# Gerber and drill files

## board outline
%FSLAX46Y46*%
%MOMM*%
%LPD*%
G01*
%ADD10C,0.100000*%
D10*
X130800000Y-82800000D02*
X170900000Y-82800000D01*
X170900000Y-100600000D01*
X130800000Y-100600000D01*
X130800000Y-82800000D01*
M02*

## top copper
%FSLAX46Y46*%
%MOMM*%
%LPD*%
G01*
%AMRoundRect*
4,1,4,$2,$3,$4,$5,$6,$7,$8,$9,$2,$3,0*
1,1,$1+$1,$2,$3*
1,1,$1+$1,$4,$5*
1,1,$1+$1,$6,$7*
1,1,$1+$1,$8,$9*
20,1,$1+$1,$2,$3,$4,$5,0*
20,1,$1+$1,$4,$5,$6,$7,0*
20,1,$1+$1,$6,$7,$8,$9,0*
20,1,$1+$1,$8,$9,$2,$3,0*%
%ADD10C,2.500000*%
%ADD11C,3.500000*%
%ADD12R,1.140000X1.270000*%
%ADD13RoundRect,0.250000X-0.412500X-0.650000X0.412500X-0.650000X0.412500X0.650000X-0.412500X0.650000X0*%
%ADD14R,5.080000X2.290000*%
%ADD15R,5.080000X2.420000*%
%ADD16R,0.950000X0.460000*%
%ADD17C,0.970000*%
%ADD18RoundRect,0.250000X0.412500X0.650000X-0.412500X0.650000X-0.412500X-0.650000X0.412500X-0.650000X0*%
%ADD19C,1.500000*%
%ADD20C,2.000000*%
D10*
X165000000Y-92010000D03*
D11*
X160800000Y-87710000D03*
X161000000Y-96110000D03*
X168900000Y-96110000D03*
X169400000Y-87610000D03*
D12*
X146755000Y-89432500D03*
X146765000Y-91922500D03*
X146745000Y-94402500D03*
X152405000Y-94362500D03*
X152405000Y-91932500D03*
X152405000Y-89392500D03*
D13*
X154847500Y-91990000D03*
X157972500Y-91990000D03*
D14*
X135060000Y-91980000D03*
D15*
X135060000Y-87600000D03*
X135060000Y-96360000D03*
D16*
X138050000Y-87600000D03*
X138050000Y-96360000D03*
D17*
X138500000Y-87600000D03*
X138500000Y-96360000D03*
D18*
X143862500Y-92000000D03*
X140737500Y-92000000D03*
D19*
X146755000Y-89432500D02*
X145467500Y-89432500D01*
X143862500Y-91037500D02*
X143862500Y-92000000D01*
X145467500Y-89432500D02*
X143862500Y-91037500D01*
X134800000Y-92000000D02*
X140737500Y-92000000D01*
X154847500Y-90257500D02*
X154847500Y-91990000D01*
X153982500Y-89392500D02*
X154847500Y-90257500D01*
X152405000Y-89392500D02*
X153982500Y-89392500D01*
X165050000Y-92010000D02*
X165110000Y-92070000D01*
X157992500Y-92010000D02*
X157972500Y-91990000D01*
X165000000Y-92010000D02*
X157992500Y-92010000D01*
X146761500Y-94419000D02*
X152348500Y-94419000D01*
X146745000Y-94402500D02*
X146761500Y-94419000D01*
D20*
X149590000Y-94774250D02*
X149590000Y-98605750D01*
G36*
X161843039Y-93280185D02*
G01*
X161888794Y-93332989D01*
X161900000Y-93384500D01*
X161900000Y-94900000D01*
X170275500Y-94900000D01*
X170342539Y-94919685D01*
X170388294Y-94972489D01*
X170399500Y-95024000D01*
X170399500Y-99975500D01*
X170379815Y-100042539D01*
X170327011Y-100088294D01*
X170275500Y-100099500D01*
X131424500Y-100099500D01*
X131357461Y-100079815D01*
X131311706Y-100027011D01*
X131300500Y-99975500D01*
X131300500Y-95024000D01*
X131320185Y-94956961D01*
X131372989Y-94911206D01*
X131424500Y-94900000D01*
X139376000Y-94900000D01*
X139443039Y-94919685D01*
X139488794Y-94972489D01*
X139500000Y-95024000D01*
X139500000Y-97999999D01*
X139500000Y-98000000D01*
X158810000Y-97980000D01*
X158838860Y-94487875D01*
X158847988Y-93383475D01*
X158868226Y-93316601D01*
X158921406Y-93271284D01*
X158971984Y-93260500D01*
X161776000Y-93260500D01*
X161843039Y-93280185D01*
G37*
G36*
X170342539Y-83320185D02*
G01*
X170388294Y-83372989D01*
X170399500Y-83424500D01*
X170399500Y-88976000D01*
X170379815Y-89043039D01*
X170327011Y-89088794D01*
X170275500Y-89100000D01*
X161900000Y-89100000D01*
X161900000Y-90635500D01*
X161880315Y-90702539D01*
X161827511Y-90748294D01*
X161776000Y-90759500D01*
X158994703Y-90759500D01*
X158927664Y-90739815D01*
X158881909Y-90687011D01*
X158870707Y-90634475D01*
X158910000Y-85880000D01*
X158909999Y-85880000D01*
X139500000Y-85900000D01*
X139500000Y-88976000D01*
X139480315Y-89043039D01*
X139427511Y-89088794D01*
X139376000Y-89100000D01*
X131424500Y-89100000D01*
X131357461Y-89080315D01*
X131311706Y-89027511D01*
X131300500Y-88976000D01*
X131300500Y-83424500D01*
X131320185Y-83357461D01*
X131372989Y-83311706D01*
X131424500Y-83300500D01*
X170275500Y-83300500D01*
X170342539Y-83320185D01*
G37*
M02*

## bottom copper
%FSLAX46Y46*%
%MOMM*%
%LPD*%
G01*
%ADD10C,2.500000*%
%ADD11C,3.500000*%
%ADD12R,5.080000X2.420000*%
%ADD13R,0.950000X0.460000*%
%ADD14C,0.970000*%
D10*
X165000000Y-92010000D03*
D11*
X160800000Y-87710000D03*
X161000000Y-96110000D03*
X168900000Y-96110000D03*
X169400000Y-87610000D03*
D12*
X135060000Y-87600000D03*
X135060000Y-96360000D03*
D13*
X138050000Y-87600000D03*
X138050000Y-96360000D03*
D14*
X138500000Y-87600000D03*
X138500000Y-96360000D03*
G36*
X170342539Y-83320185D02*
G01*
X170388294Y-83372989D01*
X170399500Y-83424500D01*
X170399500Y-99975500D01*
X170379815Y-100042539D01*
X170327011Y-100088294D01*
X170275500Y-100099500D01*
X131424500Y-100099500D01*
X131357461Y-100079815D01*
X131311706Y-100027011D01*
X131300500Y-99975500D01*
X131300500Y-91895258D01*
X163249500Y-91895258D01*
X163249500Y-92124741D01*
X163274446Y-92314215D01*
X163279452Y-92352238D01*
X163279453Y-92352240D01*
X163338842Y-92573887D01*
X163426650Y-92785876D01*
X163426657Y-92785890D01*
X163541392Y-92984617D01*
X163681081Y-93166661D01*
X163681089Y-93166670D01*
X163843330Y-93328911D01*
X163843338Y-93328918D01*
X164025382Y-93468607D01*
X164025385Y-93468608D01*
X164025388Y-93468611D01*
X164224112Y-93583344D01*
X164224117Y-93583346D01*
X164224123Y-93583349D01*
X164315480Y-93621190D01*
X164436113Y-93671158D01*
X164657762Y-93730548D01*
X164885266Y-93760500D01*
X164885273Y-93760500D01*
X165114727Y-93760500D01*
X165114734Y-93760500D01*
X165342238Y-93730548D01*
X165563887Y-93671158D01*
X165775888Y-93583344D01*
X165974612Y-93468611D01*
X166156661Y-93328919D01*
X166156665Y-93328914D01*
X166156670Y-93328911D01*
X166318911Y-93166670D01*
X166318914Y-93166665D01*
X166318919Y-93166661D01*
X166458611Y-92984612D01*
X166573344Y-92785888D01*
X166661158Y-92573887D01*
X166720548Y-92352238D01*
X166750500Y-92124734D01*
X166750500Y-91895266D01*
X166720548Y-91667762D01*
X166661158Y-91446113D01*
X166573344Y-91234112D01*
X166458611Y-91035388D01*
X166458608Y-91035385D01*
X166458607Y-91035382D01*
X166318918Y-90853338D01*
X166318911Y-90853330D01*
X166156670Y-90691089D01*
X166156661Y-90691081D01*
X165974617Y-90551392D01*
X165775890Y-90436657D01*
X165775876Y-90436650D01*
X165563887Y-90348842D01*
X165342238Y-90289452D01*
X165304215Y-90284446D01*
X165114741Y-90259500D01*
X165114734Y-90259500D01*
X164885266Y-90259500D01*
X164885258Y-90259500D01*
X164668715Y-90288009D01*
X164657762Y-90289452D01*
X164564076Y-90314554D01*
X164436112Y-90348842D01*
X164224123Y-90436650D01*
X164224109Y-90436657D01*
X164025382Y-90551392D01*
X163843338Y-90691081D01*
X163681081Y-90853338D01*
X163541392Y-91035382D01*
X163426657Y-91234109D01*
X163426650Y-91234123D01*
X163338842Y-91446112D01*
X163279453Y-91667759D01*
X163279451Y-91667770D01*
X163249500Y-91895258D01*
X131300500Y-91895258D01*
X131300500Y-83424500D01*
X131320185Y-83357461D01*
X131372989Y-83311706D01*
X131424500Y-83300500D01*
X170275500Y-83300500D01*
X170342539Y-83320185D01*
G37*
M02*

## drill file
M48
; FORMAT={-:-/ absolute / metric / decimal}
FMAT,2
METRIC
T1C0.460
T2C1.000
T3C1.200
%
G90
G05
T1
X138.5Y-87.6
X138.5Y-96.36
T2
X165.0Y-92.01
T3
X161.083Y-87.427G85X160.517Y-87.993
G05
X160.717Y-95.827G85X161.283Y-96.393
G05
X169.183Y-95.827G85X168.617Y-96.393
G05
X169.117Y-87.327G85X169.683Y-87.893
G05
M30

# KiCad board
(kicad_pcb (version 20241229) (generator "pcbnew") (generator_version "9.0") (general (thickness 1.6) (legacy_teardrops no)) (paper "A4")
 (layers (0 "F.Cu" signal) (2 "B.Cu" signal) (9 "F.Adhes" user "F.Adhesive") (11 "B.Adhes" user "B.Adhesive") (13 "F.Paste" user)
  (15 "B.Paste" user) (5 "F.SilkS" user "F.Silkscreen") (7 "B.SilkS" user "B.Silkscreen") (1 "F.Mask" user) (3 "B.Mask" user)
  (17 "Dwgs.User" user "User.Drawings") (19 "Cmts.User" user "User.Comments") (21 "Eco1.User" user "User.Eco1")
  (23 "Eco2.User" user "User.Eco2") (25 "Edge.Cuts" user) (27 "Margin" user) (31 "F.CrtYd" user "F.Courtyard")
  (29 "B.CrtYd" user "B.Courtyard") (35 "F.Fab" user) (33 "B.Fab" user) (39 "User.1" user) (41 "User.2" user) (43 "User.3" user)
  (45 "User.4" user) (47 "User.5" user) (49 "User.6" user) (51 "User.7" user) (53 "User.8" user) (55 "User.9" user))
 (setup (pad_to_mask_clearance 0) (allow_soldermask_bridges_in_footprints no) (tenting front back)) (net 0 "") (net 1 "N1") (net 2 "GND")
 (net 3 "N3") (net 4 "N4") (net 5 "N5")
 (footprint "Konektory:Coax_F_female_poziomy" (layer "F.Cu") (at 165 92.01)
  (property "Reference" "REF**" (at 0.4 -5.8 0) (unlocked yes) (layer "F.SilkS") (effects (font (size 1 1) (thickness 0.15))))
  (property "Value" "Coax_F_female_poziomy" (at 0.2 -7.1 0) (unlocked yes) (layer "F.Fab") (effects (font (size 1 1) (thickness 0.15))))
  (pad "1" thru_hole circle (at 0 0) (size 2.5 2.5) (drill 1) (layers "*.Cu" "*.Mask") (remove_unused_layers no) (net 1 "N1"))
  (pad "2" thru_hole circle (at -4.2 -4.3 315) (size 3.5 3.5) (drill oval 1.2 2) (layers "*.Cu" "*.Mask") (remove_unused_layers no)
   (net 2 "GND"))
  (pad "2" thru_hole circle (at -4 4.1 45) (size 3.5 3.5) (drill oval 1.2 2) (layers "*.Cu" "*.Mask") (remove_unused_layers no)
   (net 2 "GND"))
  (pad "2" thru_hole circle (at 3.9 4.1 315) (size 3.5 3.5) (drill oval 1.2 2) (layers "*.Cu" "*.Mask") (remove_unused_layers no)
   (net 2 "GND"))
  (pad "2" thru_hole circle (at 4.4 -4.4 45) (size 3.5 3.5) (drill oval 1.2 2) (layers "*.Cu" "*.Mask") (remove_unused_layers no)
   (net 2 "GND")))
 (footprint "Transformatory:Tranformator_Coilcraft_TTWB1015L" (layer "F.Cu") (at 146.375 88.8525)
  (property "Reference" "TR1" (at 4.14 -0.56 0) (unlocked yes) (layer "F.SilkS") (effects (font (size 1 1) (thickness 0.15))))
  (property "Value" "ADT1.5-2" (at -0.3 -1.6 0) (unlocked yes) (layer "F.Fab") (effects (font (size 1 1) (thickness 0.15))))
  (pad "1" smd rect (at 0.38 0.58) (size 1.14 1.27) (layers "F.Cu" "F.Mask" "F.Paste") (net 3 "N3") (thermal_bridge_angle 45))
  (pad "2" smd rect (at 0.39 3.07) (size 1.14 1.27) (layers "F.Cu" "F.Mask" "F.Paste") (thermal_bridge_angle 45))
  (pad "3" smd rect (at 0.37 5.55) (size 1.14 1.27) (layers "F.Cu" "F.Mask" "F.Paste") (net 2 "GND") (thermal_bridge_angle 45))
  (pad "4" smd rect (at 6.03 5.51) (size 1.14 1.27) (layers "F.Cu" "F.Mask" "F.Paste") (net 2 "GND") (thermal_bridge_angle 45))
  (pad "5" smd rect (at 6.03 3.08) (size 1.14 1.27) (layers "F.Cu" "F.Mask" "F.Paste") (thermal_bridge_angle 45))
  (pad "6" smd rect (at 6.03 0.54) (size 1.14 1.27) (layers "F.Cu" "F.Mask" "F.Paste") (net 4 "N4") (thermal_bridge_angle 45)))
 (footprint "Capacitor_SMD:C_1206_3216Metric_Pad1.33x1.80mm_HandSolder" (layer "F.Cu") (at 156.41 91.99)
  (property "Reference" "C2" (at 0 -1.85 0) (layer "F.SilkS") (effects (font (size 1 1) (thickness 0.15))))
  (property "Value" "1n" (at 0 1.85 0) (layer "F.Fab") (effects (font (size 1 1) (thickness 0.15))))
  (pad "1" smd roundrect (at -1.5625 0) (size 1.325 1.8) (layers "F.Cu" "F.Mask" "F.Paste") (roundrect_rratio 0.188679) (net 4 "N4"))
  (pad "2" smd roundrect (at 1.5625 0) (size 1.325 1.8) (layers "F.Cu" "F.Mask" "F.Paste") (roundrect_rratio 0.188679) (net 1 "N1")))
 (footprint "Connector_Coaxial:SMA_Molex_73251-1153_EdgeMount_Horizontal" (layer "F.Cu") (at 136.78 91.98)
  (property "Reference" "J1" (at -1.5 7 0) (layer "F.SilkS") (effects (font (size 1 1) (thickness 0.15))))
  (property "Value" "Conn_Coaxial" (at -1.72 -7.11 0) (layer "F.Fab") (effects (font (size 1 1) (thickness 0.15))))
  (pad "1" smd rect (at -1.72 0) (size 5.08 2.29) (layers "F.Cu" "F.Mask" "F.Paste") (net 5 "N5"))
  (pad "2" smd rect (at -1.72 -4.38) (size 5.08 2.42) (layers "F.Cu" "F.Mask" "F.Paste") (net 2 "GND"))
  (pad "2" smd rect (at -1.72 -4.38) (size 5.08 2.42) (layers "B.Cu" "B.Mask" "B.Paste") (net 2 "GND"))
  (pad "2" smd rect (at -1.72 4.38) (size 5.08 2.42) (layers "F.Cu" "F.Mask" "F.Paste") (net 2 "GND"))
  (pad "2" smd rect (at -1.72 4.38) (size 5.08 2.42) (layers "B.Cu" "B.Mask" "B.Paste") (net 2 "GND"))
  (pad "2" smd rect (at 1.27 -4.38) (size 0.95 0.46) (layers "F.Cu") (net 2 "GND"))
  (pad "2" smd rect (at 1.27 -4.38) (size 0.95 0.46) (layers "B.Cu") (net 2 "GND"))
  (pad "2" smd rect (at 1.27 4.38) (size 0.95 0.46) (layers "F.Cu") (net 2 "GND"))
  (pad "2" smd rect (at 1.27 4.38) (size 0.95 0.46) (layers "B.Cu") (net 2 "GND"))
  (pad "2" thru_hole circle (at 1.72 -4.38) (size 0.97 0.97) (drill 0.46) (layers "*.Cu") (remove_unused_layers no) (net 2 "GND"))
  (pad "2" thru_hole circle (at 1.72 4.38) (size 0.97 0.97) (drill 0.46) (layers "*.Cu") (remove_unused_layers no) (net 2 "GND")))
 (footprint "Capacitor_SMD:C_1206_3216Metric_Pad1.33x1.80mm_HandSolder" (layer "F.Cu") (at 142.3 92 180)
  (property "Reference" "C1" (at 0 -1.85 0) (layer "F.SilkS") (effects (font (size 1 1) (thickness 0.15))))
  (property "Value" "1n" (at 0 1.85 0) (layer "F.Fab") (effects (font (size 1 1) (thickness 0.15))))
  (pad "1" smd roundrect (at -1.5625 0 180) (size 1.325 1.8) (layers "F.Cu" "F.Mask" "F.Paste") (roundrect_rratio 0.188679) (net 3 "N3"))
  (pad "2" smd roundrect (at 1.5625 0 180) (size 1.325 1.8) (layers "F.Cu" "F.Mask" "F.Paste") (roundrect_rratio 0.188679) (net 5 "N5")))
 (gr_rect (start 130.8 82.8) (end 170.9 100.6) (stroke (width 0.1) (type default)) (fill no) (layer "Edge.Cuts"))
 (segment (start 146.755 89.4325) (end 145.4675 89.4325) (width 1.5) (layer "F.Cu") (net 3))
 (segment (start 143.8625 91.0375) (end 143.8625 92) (width 1.5) (layer "F.Cu") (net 3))
 (segment (start 145.4675 89.4325) (end 143.8625 91.0375) (width 1.5) (layer "F.Cu") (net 3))
 (segment (start 134.8 92) (end 140.7375 92) (width 1.5) (layer "F.Cu") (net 5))
 (segment (start 154.8475 90.2575) (end 154.8475 91.99) (width 1.5) (layer "F.Cu") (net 4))
 (segment (start 153.9825 89.3925) (end 154.8475 90.2575) (width 1.5) (layer "F.Cu") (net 4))
 (segment (start 152.405 89.3925) (end 153.9825 89.3925) (width 1.5) (layer "F.Cu") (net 4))
 (segment (start 165.05 92.01) (end 165.11 92.07) (width 1.5) (layer "F.Cu") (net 1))
 (segment (start 157.9925 92.01) (end 157.9725 91.99) (width 1.5) (layer "F.Cu") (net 1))
 (segment (start 165 92.01) (end 157.9925 92.01) (width 1.5) (layer "F.Cu") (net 1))
 (segment (start 146.7615 94.419) (end 152.3485 94.419) (width 1.5) (layer "F.Cu") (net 2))
 (segment (start 146.745 94.4025) (end 146.7615 94.419) (width 1.5) (layer "F.Cu") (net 2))
 (segment (start 149.59 94.77425) (end 149.59 98.60575) (width 2) (layer "F.Cu") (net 2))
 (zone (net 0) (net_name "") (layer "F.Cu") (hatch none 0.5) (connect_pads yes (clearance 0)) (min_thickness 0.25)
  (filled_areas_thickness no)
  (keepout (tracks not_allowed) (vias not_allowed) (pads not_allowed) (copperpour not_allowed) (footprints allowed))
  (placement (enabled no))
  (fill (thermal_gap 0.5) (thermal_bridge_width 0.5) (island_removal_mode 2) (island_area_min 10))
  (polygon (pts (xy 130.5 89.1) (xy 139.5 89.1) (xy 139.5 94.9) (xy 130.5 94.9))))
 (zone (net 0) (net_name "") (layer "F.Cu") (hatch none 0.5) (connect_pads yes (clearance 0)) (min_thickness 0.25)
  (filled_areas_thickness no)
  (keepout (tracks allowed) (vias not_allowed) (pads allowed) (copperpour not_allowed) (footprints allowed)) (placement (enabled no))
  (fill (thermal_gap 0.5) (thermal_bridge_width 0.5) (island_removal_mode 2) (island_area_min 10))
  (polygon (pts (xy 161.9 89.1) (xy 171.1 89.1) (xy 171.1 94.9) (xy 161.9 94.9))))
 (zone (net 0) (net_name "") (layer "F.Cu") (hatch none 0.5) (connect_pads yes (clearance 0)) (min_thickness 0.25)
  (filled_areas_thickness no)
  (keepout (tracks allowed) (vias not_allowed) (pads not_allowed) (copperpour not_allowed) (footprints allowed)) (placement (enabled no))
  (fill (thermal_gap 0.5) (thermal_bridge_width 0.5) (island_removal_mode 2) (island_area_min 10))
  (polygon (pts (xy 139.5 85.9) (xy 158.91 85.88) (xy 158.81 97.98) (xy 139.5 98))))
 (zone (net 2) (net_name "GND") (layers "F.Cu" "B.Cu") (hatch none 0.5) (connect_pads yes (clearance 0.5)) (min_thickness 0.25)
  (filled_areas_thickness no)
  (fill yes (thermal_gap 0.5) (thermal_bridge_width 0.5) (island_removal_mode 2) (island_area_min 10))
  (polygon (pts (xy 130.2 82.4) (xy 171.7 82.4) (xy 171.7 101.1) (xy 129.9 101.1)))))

